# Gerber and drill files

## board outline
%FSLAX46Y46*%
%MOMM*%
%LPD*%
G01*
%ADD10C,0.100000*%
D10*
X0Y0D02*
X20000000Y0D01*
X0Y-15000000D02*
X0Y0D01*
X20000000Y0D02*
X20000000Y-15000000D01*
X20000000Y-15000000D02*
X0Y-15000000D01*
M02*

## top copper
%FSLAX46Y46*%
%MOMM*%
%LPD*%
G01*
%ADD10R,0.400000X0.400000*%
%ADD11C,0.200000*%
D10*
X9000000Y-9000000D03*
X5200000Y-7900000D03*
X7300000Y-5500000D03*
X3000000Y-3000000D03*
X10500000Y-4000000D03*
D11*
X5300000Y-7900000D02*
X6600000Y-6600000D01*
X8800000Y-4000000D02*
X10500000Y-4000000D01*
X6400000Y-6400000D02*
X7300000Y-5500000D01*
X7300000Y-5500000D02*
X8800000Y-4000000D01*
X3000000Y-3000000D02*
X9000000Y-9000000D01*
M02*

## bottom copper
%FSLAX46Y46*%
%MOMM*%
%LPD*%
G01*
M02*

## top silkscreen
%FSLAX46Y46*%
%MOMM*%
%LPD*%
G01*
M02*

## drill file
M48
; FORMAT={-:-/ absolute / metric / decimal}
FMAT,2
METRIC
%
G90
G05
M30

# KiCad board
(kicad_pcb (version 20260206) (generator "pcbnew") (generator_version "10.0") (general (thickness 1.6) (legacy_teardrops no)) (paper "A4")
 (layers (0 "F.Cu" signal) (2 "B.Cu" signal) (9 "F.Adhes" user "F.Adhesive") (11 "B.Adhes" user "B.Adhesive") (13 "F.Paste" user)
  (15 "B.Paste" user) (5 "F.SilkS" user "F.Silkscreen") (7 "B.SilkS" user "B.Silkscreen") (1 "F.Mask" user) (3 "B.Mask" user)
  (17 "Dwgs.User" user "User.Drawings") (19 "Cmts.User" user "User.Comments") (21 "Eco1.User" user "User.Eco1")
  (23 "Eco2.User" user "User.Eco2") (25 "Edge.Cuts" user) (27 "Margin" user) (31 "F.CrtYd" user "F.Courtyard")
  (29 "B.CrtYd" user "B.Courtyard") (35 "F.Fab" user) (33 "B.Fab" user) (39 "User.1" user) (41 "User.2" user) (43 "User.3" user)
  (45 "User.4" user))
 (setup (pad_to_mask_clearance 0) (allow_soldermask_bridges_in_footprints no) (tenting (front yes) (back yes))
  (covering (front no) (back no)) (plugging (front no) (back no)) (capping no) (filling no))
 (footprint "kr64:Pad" (layer "F.Cu") (at 9 9)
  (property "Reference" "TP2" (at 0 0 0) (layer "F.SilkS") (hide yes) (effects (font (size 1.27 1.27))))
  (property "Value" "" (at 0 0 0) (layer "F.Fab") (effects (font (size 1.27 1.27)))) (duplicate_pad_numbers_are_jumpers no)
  (pad "1" smd rect (at 0 0) (size 0.4 0.4) (layers "F.Cu" "F.Mask" "F.Paste") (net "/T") (thermal_bridge_angle 45)))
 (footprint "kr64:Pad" (layer "F.Cu") (at 5.2 7.9)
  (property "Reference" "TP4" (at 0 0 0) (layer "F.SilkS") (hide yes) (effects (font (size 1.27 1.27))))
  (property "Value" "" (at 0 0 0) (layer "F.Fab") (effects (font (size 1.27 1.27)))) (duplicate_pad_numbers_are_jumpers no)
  (pad "1" smd rect (at 0 0) (size 0.4 0.4) (layers "F.Cu" "F.Mask" "F.Paste") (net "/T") (thermal_bridge_angle 45)))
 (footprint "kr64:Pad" (layer "F.Cu") (at 7.3 5.5)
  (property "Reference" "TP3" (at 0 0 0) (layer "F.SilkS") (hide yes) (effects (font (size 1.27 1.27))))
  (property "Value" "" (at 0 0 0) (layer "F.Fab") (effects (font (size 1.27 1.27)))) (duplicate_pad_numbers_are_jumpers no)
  (pad "1" smd rect (at 0 0) (size 0.4 0.4) (layers "F.Cu" "F.Mask" "F.Paste") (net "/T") (thermal_bridge_angle 45)))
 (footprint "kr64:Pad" (layer "F.Cu") (at 3 3)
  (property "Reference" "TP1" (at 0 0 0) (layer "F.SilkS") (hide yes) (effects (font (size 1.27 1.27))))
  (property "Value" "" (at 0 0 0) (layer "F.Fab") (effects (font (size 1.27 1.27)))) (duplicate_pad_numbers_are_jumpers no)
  (pad "1" smd rect (at 0 0) (size 0.4 0.4) (layers "F.Cu" "F.Mask" "F.Paste") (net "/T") (thermal_bridge_angle 45)))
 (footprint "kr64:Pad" (layer "F.Cu") (at 10.5 4)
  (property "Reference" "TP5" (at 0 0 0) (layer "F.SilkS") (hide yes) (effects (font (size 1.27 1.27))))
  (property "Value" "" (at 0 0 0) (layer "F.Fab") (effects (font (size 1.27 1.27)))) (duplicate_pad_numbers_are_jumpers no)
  (pad "1" smd rect (at 0 0) (size 0.4 0.4) (layers "F.Cu" "F.Mask" "F.Paste") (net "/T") (thermal_bridge_angle 45)))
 (gr_line (start 0 0) (end 20 0) (stroke (width 0.1) (type default)) (layer "Edge.Cuts"))
 (gr_line (start 0 15) (end 0 0) (stroke (width 0.1) (type default)) (layer "Edge.Cuts"))
 (gr_line (start 20 0) (end 20 15) (stroke (width 0.1) (type default)) (layer "Edge.Cuts"))
 (gr_line (start 20 15) (end 0 15) (stroke (width 0.1) (type default)) (layer "Edge.Cuts"))
 (segment (start 5.3 7.9) (end 6.6 6.6) (width 0.2) (layer "F.Cu") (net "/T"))
 (segment (start 8.8 4) (end 10.5 4) (width 0.2) (layer "F.Cu") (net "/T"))
 (segment (start 6.4 6.4) (end 7.3 5.5) (width 0.2) (layer "F.Cu") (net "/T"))
 (segment (start 7.3 5.5) (end 8.8 4) (width 0.2) (layer "F.Cu") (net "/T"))
 (segment (start 3 3) (end 9 9) (width 0.2) (layer "F.Cu") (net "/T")))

